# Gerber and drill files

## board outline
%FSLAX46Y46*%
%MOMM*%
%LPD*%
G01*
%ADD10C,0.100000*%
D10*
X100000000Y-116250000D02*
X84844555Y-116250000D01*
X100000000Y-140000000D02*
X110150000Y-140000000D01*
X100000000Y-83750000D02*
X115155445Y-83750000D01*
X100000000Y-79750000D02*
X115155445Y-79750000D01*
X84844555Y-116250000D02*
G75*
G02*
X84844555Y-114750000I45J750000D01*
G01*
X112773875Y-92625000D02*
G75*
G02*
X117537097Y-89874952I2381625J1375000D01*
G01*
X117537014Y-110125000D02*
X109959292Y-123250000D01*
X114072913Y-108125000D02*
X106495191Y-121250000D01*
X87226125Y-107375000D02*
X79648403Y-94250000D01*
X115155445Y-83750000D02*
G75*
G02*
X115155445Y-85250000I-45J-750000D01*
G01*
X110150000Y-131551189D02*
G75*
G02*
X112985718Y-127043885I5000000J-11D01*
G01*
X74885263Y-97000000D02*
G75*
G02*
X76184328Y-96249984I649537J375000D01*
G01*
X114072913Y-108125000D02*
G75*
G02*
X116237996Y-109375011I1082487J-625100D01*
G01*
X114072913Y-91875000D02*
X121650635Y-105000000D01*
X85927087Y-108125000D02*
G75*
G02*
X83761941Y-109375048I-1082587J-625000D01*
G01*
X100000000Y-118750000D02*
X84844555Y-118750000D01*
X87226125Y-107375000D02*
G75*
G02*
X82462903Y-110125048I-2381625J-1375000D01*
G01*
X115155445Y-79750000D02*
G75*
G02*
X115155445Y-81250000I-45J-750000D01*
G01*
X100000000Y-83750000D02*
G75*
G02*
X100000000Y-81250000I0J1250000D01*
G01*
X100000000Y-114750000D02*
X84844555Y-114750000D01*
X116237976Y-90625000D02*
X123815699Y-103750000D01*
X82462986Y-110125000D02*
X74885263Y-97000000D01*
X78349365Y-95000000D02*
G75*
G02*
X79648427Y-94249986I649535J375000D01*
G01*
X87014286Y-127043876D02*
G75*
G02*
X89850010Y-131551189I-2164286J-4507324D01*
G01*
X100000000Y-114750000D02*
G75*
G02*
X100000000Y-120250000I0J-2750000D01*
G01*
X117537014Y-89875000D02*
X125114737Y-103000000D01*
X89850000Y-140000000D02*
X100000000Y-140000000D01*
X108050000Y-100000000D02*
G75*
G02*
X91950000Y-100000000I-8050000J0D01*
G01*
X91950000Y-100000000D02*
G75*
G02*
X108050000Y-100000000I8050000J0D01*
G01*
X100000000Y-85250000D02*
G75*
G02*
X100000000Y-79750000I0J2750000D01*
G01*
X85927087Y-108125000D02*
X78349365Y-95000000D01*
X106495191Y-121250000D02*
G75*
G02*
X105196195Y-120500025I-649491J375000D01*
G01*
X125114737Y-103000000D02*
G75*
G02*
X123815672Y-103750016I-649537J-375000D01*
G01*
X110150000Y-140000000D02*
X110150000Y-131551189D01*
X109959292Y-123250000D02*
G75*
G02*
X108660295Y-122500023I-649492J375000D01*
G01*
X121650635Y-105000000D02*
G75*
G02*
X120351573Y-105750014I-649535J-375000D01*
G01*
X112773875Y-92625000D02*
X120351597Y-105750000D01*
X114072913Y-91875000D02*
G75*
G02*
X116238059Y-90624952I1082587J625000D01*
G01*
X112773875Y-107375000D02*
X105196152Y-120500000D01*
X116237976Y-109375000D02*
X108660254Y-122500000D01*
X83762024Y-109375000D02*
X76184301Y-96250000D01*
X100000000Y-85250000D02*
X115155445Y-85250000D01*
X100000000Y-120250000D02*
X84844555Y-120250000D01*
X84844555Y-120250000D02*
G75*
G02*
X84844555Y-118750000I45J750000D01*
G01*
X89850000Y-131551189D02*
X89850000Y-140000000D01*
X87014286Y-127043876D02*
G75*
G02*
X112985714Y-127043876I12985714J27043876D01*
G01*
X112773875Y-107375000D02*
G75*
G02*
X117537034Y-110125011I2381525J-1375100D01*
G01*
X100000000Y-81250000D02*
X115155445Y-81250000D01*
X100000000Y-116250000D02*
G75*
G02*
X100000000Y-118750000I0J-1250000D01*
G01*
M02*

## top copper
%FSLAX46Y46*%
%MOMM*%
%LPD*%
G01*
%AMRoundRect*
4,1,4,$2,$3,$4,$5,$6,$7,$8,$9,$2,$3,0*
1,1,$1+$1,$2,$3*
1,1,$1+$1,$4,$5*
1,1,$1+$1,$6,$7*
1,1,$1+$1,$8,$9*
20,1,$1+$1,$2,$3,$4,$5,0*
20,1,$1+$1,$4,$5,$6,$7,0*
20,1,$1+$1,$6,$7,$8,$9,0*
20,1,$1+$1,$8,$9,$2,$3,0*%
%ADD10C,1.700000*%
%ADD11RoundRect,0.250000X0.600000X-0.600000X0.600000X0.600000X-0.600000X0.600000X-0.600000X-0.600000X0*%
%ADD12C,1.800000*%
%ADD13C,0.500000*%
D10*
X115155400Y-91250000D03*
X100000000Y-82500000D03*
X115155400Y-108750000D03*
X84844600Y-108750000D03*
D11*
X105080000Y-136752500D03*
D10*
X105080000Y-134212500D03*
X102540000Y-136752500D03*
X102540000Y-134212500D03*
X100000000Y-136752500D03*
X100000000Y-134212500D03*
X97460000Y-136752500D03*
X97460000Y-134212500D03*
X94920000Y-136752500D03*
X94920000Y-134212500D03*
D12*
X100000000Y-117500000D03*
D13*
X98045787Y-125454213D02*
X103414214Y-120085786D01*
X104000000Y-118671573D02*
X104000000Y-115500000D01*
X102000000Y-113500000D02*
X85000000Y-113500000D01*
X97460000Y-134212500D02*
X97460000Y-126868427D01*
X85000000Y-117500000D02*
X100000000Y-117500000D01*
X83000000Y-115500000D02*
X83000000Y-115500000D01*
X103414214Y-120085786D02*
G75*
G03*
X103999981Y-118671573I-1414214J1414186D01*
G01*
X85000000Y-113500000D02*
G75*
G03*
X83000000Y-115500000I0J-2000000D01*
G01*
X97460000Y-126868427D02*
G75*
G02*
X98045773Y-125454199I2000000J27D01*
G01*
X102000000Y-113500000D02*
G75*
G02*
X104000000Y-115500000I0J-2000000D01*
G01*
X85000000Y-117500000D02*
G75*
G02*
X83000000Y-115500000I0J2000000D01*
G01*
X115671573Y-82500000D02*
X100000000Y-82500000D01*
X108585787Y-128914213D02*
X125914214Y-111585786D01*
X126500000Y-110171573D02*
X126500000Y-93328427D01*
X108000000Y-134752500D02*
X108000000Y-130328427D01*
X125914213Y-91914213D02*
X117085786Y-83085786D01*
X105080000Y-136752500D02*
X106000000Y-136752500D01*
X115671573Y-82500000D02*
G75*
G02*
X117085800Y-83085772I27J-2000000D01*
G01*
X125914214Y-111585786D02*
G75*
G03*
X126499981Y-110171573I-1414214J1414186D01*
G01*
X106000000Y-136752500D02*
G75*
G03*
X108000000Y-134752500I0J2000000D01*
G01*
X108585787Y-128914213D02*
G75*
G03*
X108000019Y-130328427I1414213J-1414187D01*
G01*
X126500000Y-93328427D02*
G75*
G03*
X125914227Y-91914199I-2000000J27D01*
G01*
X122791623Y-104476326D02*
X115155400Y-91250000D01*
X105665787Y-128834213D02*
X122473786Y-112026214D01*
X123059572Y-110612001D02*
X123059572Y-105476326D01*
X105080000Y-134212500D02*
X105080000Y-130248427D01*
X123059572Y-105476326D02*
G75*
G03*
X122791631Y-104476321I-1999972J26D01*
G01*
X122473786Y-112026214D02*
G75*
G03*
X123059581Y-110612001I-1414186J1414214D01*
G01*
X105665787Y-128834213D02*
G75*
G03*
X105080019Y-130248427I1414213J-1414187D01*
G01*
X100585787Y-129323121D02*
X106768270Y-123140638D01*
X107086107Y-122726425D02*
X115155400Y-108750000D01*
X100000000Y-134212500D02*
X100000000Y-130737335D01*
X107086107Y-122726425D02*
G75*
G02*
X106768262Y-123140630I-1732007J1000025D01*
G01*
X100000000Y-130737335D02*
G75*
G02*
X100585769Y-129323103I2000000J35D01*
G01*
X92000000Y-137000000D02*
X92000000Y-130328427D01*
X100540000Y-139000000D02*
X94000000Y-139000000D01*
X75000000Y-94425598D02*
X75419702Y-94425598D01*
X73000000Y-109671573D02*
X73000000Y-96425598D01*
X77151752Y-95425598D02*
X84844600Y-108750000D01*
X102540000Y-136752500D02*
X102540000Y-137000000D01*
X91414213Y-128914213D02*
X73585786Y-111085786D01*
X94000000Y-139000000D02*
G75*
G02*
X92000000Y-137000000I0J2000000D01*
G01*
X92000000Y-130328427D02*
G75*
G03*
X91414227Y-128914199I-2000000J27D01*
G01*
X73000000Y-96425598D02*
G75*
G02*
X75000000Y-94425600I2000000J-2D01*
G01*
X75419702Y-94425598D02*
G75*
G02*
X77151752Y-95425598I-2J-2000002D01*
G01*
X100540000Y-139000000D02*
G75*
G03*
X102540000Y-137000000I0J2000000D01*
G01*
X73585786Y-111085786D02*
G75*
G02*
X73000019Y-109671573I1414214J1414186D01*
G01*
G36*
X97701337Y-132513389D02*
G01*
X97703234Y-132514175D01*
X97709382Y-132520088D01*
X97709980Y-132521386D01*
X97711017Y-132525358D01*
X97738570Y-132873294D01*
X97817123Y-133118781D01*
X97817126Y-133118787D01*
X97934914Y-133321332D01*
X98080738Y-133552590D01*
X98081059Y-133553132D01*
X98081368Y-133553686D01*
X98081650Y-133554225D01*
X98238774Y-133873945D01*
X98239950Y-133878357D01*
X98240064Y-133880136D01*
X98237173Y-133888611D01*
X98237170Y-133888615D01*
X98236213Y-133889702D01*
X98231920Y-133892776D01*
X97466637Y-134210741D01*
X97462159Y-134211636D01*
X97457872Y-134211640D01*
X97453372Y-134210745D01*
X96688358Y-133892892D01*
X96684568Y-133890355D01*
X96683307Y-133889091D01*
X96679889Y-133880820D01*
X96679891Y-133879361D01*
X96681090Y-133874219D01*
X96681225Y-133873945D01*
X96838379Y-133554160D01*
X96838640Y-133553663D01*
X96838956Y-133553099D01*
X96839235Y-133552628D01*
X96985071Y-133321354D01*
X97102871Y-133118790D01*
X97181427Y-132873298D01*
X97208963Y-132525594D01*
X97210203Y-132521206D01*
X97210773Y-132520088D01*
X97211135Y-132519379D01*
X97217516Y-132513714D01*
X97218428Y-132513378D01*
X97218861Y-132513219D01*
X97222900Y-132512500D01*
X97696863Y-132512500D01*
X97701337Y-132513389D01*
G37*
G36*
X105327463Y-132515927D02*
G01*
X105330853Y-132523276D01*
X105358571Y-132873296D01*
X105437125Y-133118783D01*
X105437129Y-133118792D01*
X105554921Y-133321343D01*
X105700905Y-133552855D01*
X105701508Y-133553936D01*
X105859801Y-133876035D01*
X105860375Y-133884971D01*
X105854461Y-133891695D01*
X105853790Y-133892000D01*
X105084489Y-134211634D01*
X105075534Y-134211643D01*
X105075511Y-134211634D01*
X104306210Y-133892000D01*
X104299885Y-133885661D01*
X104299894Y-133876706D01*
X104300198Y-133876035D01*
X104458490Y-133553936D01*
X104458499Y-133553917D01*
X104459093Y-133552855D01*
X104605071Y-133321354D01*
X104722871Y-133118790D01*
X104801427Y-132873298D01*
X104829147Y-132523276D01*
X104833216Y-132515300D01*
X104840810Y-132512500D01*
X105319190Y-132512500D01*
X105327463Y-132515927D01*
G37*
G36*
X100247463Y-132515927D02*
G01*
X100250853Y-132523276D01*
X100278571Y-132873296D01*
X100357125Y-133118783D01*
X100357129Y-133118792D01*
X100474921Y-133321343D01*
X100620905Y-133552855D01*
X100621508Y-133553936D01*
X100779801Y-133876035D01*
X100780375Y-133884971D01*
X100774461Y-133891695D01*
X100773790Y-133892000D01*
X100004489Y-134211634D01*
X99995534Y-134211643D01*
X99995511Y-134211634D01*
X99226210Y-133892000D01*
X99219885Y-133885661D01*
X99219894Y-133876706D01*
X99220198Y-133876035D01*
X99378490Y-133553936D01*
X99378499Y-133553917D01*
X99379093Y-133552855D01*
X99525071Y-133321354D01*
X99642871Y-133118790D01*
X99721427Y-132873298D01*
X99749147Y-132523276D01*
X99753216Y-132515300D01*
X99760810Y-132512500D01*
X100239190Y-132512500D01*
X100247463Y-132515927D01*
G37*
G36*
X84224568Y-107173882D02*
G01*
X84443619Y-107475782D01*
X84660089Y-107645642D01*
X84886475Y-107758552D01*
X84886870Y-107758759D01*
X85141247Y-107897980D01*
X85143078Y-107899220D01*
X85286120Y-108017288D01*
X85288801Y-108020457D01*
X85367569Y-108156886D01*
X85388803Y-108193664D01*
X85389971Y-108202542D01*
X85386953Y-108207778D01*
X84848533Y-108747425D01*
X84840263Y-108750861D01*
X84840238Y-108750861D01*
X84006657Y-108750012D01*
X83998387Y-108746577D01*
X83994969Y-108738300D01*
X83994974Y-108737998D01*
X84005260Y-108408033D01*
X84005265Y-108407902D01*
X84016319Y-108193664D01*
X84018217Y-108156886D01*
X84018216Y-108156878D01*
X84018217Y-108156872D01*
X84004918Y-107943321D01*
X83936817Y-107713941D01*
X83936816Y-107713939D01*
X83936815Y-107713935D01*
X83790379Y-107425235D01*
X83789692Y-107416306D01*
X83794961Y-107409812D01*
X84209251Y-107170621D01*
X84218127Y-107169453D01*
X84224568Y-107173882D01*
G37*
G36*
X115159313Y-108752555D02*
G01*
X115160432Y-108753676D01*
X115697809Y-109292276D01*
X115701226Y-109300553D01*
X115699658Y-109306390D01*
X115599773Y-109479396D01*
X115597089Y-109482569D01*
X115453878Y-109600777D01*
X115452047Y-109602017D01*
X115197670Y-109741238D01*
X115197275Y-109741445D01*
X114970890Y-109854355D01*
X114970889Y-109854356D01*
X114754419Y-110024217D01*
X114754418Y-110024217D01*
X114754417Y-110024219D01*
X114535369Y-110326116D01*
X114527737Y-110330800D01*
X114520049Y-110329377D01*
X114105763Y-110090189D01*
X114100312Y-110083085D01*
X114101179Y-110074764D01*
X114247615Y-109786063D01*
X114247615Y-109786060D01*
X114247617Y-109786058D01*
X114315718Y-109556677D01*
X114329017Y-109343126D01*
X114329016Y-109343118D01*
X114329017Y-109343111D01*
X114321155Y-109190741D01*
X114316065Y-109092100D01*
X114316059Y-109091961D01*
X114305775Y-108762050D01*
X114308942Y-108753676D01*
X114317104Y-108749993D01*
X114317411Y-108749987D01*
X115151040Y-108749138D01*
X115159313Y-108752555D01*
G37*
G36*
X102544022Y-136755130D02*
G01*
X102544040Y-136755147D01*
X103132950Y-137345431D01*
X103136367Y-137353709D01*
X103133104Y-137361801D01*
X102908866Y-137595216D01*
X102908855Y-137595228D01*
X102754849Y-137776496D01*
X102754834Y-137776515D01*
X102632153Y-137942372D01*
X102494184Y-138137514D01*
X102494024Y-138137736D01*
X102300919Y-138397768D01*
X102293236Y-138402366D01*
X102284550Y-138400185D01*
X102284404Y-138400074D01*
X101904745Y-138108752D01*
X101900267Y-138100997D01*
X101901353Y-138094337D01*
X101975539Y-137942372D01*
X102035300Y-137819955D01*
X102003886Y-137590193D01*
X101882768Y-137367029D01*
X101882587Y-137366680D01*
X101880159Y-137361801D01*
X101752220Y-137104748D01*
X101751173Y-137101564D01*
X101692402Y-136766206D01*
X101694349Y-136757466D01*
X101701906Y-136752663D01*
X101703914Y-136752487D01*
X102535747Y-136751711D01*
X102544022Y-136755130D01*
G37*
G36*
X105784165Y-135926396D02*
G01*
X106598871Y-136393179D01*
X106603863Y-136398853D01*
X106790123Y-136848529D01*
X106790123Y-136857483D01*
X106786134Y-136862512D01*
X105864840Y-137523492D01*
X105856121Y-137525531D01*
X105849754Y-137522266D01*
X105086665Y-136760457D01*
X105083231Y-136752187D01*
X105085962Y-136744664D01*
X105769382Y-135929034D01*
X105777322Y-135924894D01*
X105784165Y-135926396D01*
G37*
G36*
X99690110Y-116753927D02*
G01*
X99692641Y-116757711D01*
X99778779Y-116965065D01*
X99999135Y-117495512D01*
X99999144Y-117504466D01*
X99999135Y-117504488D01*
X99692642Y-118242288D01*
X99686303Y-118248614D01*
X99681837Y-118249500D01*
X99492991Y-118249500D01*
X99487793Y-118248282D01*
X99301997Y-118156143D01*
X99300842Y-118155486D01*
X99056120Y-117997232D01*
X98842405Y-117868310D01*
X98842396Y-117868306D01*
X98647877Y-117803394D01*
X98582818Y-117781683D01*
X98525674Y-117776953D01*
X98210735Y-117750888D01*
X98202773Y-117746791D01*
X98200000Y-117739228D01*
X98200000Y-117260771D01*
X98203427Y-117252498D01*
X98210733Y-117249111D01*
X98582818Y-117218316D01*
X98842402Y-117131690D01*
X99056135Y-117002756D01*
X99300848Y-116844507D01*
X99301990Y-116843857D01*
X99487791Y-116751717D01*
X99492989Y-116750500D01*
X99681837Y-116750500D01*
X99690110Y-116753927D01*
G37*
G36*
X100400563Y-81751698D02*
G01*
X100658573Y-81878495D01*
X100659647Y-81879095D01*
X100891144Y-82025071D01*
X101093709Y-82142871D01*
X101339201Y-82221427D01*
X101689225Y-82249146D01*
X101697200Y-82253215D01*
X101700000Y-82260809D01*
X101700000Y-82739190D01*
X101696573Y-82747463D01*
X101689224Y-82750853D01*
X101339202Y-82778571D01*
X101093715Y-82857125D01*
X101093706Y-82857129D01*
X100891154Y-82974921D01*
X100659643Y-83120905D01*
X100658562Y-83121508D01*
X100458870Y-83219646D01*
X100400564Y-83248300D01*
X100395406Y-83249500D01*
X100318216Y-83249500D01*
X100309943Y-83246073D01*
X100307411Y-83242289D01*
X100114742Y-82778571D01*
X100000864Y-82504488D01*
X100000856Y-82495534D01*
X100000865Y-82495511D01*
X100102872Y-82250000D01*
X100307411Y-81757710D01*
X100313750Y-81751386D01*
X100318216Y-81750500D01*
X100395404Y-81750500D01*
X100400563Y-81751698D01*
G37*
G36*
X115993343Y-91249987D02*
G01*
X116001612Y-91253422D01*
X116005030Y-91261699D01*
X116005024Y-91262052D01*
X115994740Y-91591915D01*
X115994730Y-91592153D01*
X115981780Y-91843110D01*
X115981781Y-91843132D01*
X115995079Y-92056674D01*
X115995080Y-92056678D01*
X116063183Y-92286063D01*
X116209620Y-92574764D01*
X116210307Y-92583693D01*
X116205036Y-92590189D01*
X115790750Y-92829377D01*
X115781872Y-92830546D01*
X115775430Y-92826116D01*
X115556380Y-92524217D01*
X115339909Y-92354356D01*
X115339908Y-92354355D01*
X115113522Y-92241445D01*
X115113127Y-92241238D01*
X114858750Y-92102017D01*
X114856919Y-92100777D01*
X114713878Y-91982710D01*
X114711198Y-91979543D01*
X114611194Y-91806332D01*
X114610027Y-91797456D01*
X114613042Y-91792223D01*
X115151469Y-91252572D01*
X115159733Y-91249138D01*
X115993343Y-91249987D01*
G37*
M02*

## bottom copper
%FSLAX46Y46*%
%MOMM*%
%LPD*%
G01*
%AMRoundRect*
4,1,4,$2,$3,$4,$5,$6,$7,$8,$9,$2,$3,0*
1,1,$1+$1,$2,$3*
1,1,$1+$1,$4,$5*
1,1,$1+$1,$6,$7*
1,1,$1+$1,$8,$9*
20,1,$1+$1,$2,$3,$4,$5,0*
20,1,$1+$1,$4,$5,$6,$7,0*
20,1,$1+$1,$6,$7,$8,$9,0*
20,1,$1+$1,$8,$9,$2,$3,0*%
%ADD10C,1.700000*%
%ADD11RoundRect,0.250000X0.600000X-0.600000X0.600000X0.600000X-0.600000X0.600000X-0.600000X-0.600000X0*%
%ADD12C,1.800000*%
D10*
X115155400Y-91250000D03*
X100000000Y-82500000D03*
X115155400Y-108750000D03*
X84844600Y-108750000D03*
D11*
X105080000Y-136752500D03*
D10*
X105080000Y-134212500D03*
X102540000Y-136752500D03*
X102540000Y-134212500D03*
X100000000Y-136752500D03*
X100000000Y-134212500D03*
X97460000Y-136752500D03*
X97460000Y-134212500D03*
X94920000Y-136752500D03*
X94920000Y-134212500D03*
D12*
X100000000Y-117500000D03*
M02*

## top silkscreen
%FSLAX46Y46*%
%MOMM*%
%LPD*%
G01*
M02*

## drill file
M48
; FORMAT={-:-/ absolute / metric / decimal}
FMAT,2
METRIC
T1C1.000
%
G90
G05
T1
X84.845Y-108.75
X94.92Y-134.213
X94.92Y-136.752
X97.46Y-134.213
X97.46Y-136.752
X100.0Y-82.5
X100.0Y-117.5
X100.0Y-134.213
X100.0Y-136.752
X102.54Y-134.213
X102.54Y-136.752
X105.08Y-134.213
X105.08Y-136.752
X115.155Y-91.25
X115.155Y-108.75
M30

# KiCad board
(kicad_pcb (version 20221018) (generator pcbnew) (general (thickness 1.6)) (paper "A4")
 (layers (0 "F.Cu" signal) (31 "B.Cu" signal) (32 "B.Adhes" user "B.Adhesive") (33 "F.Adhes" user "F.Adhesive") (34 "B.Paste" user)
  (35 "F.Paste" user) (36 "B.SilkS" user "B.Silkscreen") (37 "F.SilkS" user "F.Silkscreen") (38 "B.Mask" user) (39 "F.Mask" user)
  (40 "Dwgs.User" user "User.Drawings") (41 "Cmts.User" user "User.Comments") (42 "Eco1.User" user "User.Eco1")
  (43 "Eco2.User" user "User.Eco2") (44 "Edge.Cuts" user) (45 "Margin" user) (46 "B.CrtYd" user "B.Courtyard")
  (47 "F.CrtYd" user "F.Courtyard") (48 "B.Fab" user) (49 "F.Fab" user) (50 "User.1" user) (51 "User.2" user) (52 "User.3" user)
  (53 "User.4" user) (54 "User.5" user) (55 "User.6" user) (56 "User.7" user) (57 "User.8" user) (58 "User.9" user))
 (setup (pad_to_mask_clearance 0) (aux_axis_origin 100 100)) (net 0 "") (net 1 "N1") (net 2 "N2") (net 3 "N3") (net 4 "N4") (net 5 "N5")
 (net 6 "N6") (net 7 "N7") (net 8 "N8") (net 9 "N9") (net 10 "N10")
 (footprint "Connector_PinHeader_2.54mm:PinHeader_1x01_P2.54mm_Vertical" (layer "B.Cu") (at 115.1554 91.25 180)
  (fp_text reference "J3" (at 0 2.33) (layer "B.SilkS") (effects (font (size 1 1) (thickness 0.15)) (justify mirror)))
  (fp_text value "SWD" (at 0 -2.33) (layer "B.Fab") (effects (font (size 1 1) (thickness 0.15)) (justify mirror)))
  (pad "1" thru_hole circle (at 0 0 180) (size 1.7 1.7) (drill 1) (layers "*.Cu" "*.Mask") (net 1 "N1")))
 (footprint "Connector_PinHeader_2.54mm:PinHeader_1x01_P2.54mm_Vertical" (layer "B.Cu") (at 100 82.5 180)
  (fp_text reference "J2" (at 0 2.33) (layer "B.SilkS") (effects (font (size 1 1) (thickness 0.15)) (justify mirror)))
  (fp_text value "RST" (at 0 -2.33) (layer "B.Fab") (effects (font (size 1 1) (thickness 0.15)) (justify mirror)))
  (pad "1" thru_hole circle (at 0 0 180) (size 1.7 1.7) (drill 1) (layers "*.Cu" "*.Mask") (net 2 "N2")))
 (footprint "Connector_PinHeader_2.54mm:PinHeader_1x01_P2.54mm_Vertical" (layer "B.Cu") (at 115.1554 108.75 180)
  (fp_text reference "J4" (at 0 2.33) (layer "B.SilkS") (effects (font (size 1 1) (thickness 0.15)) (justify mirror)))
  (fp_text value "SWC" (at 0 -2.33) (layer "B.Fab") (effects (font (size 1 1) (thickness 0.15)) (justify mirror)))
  (pad "1" thru_hole circle (at 0 0 180) (size 1.7 1.7) (drill 1) (layers "*.Cu" "*.Mask") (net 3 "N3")))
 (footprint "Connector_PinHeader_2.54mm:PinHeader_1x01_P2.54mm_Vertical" (layer "B.Cu") (at 84.8446 108.75 180)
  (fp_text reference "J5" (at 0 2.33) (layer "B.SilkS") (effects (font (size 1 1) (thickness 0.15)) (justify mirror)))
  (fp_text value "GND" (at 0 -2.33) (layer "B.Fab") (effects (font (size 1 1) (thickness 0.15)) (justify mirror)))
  (pad "1" thru_hole circle (at 0 0 180) (size 1.7 1.7) (drill 1) (layers "*.Cu" "*.Mask") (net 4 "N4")))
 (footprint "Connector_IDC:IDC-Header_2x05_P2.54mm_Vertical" (layer "B.Cu") (at 105.08 136.7525 90)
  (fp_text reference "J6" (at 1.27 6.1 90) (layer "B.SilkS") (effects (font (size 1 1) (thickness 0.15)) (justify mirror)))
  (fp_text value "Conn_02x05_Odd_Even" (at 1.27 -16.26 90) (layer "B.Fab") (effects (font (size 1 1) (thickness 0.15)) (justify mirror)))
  (pad "1" thru_hole roundrect (at 0 0 90) (size 1.7 1.7) (drill 1) (layers "*.Cu" "*.Mask") (roundrect_rratio 0.1470588235) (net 2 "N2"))
  (pad "2" thru_hole circle (at 2.54 0 90) (size 1.7 1.7) (drill 1) (layers "*.Cu" "*.Mask") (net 1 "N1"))
  (pad "3" thru_hole circle (at 0 -2.54 90) (size 1.7 1.7) (drill 1) (layers "*.Cu" "*.Mask") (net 4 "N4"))
  (pad "4" thru_hole circle (at 2.54 -2.54 90) (size 1.7 1.7) (drill 1) (layers "*.Cu" "*.Mask") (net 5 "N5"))
  (pad "5" thru_hole circle (at 0 -5.08 90) (size 1.7 1.7) (drill 1) (layers "*.Cu" "*.Mask") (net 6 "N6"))
  (pad "6" thru_hole circle (at 2.54 -5.08 90) (size 1.7 1.7) (drill 1) (layers "*.Cu" "*.Mask") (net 3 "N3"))
  (pad "7" thru_hole circle (at 0 -7.62 90) (size 1.7 1.7) (drill 1) (layers "*.Cu" "*.Mask") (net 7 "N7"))
  (pad "8" thru_hole circle (at 2.54 -7.62 90) (size 1.7 1.7) (drill 1) (layers "*.Cu" "*.Mask") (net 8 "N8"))
  (pad "9" thru_hole circle (at 0 -10.16 90) (size 1.7 1.7) (drill 1) (layers "*.Cu" "*.Mask") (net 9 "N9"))
  (pad "10" thru_hole circle (at 2.54 -10.16 90) (size 1.7 1.7) (drill 1) (layers "*.Cu" "*.Mask") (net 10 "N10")))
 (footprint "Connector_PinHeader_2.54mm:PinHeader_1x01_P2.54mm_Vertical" (layer "B.Cu") (at 100 117.5 180)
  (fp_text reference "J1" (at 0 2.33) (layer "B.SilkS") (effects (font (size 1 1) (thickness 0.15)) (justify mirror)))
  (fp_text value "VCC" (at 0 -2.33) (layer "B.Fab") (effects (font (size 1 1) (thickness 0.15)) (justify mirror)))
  (pad "1" thru_hole circle (at 0 0 180) (size 1.8 1.8) (drill 1) (layers "*.Cu" "*.Mask") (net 8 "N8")))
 (gr_line (start 100 116.25) (end 84.844555 116.25) (stroke (width 0.1) (type solid)) (layer "Edge.Cuts"))
 (gr_line (start 100 140) (end 110.15 140) (stroke (width 0.1) (type solid)) (layer "Edge.Cuts"))
 (gr_line (start 100 83.75) (end 115.155445 83.75) (stroke (width 0.1) (type solid)) (layer "Edge.Cuts"))
 (gr_line (start 100 79.75) (end 115.155445 79.75) (stroke (width 0.1) (type solid)) (layer "Edge.Cuts"))
 (gr_arc (start 84.844555 116.25) (mid 84.0946 115.5) (end 84.844555 114.75) (stroke (width 0.1) (type solid)) (layer "Edge.Cuts"))
 (gr_arc (start 112.773875 92.625) (mid 113.780419 88.868464) (end 117.537014 89.875) (stroke (width 0.1) (type solid)) (layer "Edge.Cuts"))
 (gr_line (start 117.537014 110.125) (end 109.959292 123.25) (stroke (width 0.1) (type solid)) (layer "Edge.Cuts"))
 (gr_line (start 114.072913 108.125) (end 106.495191 121.25) (stroke (width 0.1) (type solid)) (layer "Edge.Cuts"))
 (gr_line (start 87.226125 107.375) (end 79.648403 94.25) (stroke (width 0.1) (type solid)) (layer "Edge.Cuts"))
 (gr_arc (start 115.155445 83.75) (mid 115.9054 84.5) (end 115.155445 85.25) (stroke (width 0.1) (type solid)) (layer "Edge.Cuts"))
 (gr_arc (start 110.15 131.551189) (mid 110.917899 128.888622) (end 112.985714 127.043876) (stroke (width 0.1) (type solid))
  (layer "Edge.Cuts"))
 (gr_arc (start 74.885263 97) (mid 75.159792 95.975468) (end 76.184301 96.25) (stroke (width 0.1) (type solid)) (layer "Edge.Cuts"))
 (gr_arc (start 114.072913 108.125) (mid 115.780381 107.667502) (end 116.237976 109.375) (stroke (width 0.1) (type solid))
  (layer "Edge.Cuts"))
 (gr_line (start 114.072913 91.875) (end 121.650635 105) (stroke (width 0.1) (type solid)) (layer "Edge.Cuts"))
 (gr_arc (start 85.927087 108.125) (mid 85.469581 109.832498) (end 83.762024 109.375) (stroke (width 0.1) (type solid)) (layer "Edge.Cuts"))
 (gr_line (start 100 118.75) (end 84.844555 118.75) (stroke (width 0.1) (type solid)) (layer "Edge.Cuts"))
 (gr_arc (start 87.226125 107.375) (mid 86.219581 111.131536) (end 82.462986 110.125) (stroke (width 0.1) (type solid)) (layer "Edge.Cuts"))
 (gr_arc (start 115.155445 79.75) (mid 115.9054 80.5) (end 115.155445 81.25) (stroke (width 0.1) (type solid)) (layer "Edge.Cuts"))
 (gr_arc (start 100 83.75) (mid 98.75 82.5) (end 100 81.25) (stroke (width 0.1) (type solid)) (layer "Edge.Cuts"))
 (gr_line (start 100 114.75) (end 84.844555 114.75) (stroke (width 0.1) (type solid)) (layer "Edge.Cuts"))
 (gr_line (start 116.237976 90.625) (end 123.815699 103.75) (stroke (width 0.1) (type solid)) (layer "Edge.Cuts"))
 (gr_line (start 82.462986 110.125) (end 74.885263 97) (stroke (width 0.1) (type solid)) (layer "Edge.Cuts"))
 (gr_arc (start 78.349365 95) (mid 78.623893 93.975469) (end 79.648403 94.25) (stroke (width 0.1) (type solid)) (layer "Edge.Cuts"))
 (gr_arc (start 87.014286 127.043876) (mid 89.08211 128.888617) (end 89.85 131.551189) (stroke (width 0.1) (type solid)) (layer "Edge.Cuts"))
 (gr_arc (start 100 114.75) (mid 102.75 117.5) (end 100 120.25) (stroke (width 0.1) (type solid)) (layer "Edge.Cuts"))
 (gr_line (start 117.537014 89.875) (end 125.114737 103) (stroke (width 0.1) (type solid)) (layer "Edge.Cuts"))
 (gr_line (start 89.85 140) (end 100 140) (stroke (width 0.1) (type solid)) (layer "Edge.Cuts"))
 (gr_circle (center 100 100) (end 108.05 100) (stroke (width 0.1) (type solid)) (fill none) (layer "Edge.Cuts"))
 (gr_arc (start 100 85.25) (mid 97.25 82.5) (end 100 79.75) (stroke (width 0.1) (type solid)) (layer "Edge.Cuts"))
 (gr_line (start 85.927087 108.125) (end 78.349365 95) (stroke (width 0.1) (type solid)) (layer "Edge.Cuts"))
 (gr_arc (start 106.495191 121.25) (mid 105.470712 121.524498) (end 105.196152 120.5) (stroke (width 0.1) (type solid)) (layer "Edge.Cuts"))
 (gr_arc (start 125.114737 103) (mid 124.840208 104.024532) (end 123.815699 103.75) (stroke (width 0.1) (type solid)) (layer "Edge.Cuts"))
 (gr_line (start 110.15 140) (end 110.15 131.551189) (stroke (width 0.1) (type solid)) (layer "Edge.Cuts"))
 (gr_arc (start 109.959292 123.25) (mid 108.934812 123.524499) (end 108.660254 122.5) (stroke (width 0.1) (type solid)) (layer "Edge.Cuts"))
 (gr_arc (start 121.650635 105) (mid 121.376107 106.024531) (end 120.351597 105.75) (stroke (width 0.1) (type solid)) (layer "Edge.Cuts"))
 (gr_line (start 112.773875 92.625) (end 120.351597 105.75) (stroke (width 0.1) (type solid)) (layer "Edge.Cuts"))
 (gr_arc (start 114.072913 91.875) (mid 114.530419 90.167502) (end 116.237976 90.625) (stroke (width 0.1) (type solid)) (layer "Edge.Cuts"))
 (gr_line (start 112.773875 107.375) (end 105.196152 120.5) (stroke (width 0.1) (type solid)) (layer "Edge.Cuts"))
 (gr_line (start 116.237976 109.375) (end 108.660254 122.5) (stroke (width 0.1) (type solid)) (layer "Edge.Cuts"))
 (gr_line (start 83.762024 109.375) (end 76.184301 96.25) (stroke (width 0.1) (type solid)) (layer "Edge.Cuts"))
 (gr_line (start 100 85.25) (end 115.155445 85.25) (stroke (width 0.1) (type solid)) (layer "Edge.Cuts"))
 (gr_line (start 100 120.25) (end 84.844555 120.25) (stroke (width 0.1) (type solid)) (layer "Edge.Cuts"))
 (gr_arc (start 84.844555 120.25) (mid 84.0946 119.5) (end 84.844555 118.75) (stroke (width 0.1) (type solid)) (layer "Edge.Cuts"))
 (gr_line (start 89.85 131.551189) (end 89.85 140) (stroke (width 0.1) (type solid)) (layer "Edge.Cuts"))
 (gr_arc (start 87.014286 127.043876) (mid 100 70) (end 112.985714 127.043876) (stroke (width 0.1) (type solid)) (layer "Edge.Cuts"))
 (gr_arc (start 112.773875 107.375) (mid 116.530381 106.368464) (end 117.537014 110.125) (stroke (width 0.1) (type solid))
  (layer "Edge.Cuts"))
 (gr_line (start 100 81.25) (end 115.155445 81.25) (stroke (width 0.1) (type solid)) (layer "Edge.Cuts"))
 (gr_arc (start 100 116.25) (mid 101.25 117.5) (end 100 118.75) (stroke (width 0.1) (type solid)) (layer "Edge.Cuts"))
 (segment (start 98.045787 125.454213) (end 103.414214 120.085786) (width 0.5) (layer "F.Cu") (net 8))
 (segment (start 104 118.671573) (end 104 115.5) (width 0.5) (layer "F.Cu") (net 8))
 (segment (start 102 113.5) (end 85 113.5) (width 0.5) (layer "F.Cu") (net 8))
 (segment (start 97.46 134.2125) (end 97.46 126.868427) (width 0.5) (layer "F.Cu") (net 8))
 (segment (start 85 117.5) (end 100 117.5) (width 0.5) (layer "F.Cu") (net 8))
 (segment (start 83 115.5) (end 83 115.5) (width 0.5) (layer "F.Cu") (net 8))
 (arc (start 103.414214 120.085786) (mid 103.847759 119.43694) (end 104 118.671573) (width 0.5) (layer "F.Cu") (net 8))
 (arc (start 85 113.5) (mid 83.585786 114.085786) (end 83 115.5) (width 0.5) (layer "F.Cu") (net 8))
 (arc (start 97.46 126.868427) (mid 97.612241 126.10306) (end 98.045787 125.454213) (width 0.5) (layer "F.Cu") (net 8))
 (arc (start 102 113.5) (mid 103.414214 114.085786) (end 104 115.5) (width 0.5) (layer "F.Cu") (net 8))
 (arc (start 85 117.5) (mid 83.585786 116.914214) (end 83 115.5) (width 0.5) (layer "F.Cu") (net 8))
 (segment (start 115.671573 82.5) (end 100 82.5) (width 0.5) (layer "F.Cu") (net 2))
 (segment (start 108.585787 128.914213) (end 125.914214 111.585786) (width 0.5) (layer "F.Cu") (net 2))
 (segment (start 126.5 110.171573) (end 126.5 93.328427) (width 0.5) (layer "F.Cu") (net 2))
 (segment (start 108 134.7525) (end 108 130.328427) (width 0.5) (layer "F.Cu") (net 2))
 (segment (start 125.914213 91.914213) (end 117.085786 83.085786) (width 0.5) (layer "F.Cu") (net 2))
 (segment (start 105.08 136.7525) (end 106 136.7525) (width 0.5) (layer "F.Cu") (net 2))
 (arc (start 115.671573 82.5) (mid 116.43694 82.652241) (end 117.085786 83.085786) (width 0.5) (layer "F.Cu") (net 2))
 (arc (start 125.914214 111.585786) (mid 126.347759 110.93694) (end 126.5 110.171573) (width 0.5) (layer "F.Cu") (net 2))
 (arc (start 106 136.7525) (mid 107.414214 136.166714) (end 108 134.7525) (width 0.5) (layer "F.Cu") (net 2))
 (arc (start 108.585787 128.914213) (mid 108.152241 129.56306) (end 108 130.328427) (width 0.5) (layer "F.Cu") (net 2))
 (arc (start 126.5 93.328427) (mid 126.347759 92.56306) (end 125.914213 91.914213) (width 0.5) (layer "F.Cu") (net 2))
 (segment (start 122.791623 104.476326) (end 115.1554 91.25) (width 0.5) (layer "F.Cu") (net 1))
 (segment (start 105.665787 128.834213) (end 122.473786 112.026214) (width 0.5) (layer "F.Cu") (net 1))
 (segment (start 123.059572 110.612001) (end 123.059572 105.476326) (width 0.5) (layer "F.Cu") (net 1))
 (segment (start 105.08 134.2125) (end 105.08 130.248427) (width 0.5) (layer "F.Cu") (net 1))
 (arc (start 123.059572 105.476326) (mid 122.991424 104.958688) (end 122.791623 104.476326) (width 0.5) (layer "F.Cu") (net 1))
 (arc (start 122.473786 112.026214) (mid 122.907331 111.377368) (end 123.059572 110.612001) (width 0.5) (layer "F.Cu") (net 1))
 (arc (start 105.665787 128.834213) (mid 105.232241 129.48306) (end 105.08 130.248427) (width 0.5) (layer "F.Cu") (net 1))
 (segment (start 100.585787 129.323121) (end 106.76827 123.140638) (width 0.5) (layer "F.Cu") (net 3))
 (segment (start 107.086107 122.726425) (end 115.1554 108.75) (width 0.5) (layer "F.Cu") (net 3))
 (segment (start 100 134.2125) (end 100 130.737335) (width 0.5) (layer "F.Cu") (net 3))
 (arc (start 107.086107 122.726425) (mid 106.940763 122.943948) (end 106.76827 123.140638) (width 0.5) (layer "F.Cu") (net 3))
 (arc (start 100 130.737335) (mid 100.152241 129.971968) (end 100.585787 129.323121) (width 0.5) (layer "F.Cu") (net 3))
 (segment (start 92 137) (end 92 130.328427) (width 0.5) (layer "F.Cu") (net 4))
 (segment (start 100.54 139) (end 94 139) (width 0.5) (layer "F.Cu") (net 4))
 (segment (start 75 94.425598) (end 75.419702 94.425598) (width 0.5) (layer "F.Cu") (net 4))
 (segment (start 73 109.671573) (end 73 96.425598) (width 0.5) (layer "F.Cu") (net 4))
 (segment (start 77.151752 95.425598) (end 84.8446 108.75) (width 0.5) (layer "F.Cu") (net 4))
 (segment (start 102.54 136.7525) (end 102.54 137) (width 0.5) (layer "F.Cu") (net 4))
 (segment (start 91.414213 128.914213) (end 73.585786 111.085786) (width 0.5) (layer "F.Cu") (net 4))
 (arc (start 94 139) (mid 92.585786 138.414214) (end 92 137) (width 0.5) (layer "F.Cu") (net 4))
 (arc (start 92 130.328427) (mid 91.847759 129.56306) (end 91.414213 128.914213) (width 0.5) (layer "F.Cu") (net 4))
 (arc (start 73 96.425598) (mid 73.585786 95.011384) (end 75 94.425598) (width 0.5) (layer "F.Cu") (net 4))
 (arc (start 75.419702 94.425598) (mid 76.419702 94.693547) (end 77.151752 95.425598) (width 0.5) (layer "F.Cu") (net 4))
 (arc (start 100.54 139) (mid 101.954214 138.414214) (end 102.54 137) (width 0.5) (layer "F.Cu") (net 4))
 (arc (start 73.585786 111.085786) (mid 73.152241 110.43694) (end 73 109.671573) (width 0.5) (layer "F.Cu") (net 4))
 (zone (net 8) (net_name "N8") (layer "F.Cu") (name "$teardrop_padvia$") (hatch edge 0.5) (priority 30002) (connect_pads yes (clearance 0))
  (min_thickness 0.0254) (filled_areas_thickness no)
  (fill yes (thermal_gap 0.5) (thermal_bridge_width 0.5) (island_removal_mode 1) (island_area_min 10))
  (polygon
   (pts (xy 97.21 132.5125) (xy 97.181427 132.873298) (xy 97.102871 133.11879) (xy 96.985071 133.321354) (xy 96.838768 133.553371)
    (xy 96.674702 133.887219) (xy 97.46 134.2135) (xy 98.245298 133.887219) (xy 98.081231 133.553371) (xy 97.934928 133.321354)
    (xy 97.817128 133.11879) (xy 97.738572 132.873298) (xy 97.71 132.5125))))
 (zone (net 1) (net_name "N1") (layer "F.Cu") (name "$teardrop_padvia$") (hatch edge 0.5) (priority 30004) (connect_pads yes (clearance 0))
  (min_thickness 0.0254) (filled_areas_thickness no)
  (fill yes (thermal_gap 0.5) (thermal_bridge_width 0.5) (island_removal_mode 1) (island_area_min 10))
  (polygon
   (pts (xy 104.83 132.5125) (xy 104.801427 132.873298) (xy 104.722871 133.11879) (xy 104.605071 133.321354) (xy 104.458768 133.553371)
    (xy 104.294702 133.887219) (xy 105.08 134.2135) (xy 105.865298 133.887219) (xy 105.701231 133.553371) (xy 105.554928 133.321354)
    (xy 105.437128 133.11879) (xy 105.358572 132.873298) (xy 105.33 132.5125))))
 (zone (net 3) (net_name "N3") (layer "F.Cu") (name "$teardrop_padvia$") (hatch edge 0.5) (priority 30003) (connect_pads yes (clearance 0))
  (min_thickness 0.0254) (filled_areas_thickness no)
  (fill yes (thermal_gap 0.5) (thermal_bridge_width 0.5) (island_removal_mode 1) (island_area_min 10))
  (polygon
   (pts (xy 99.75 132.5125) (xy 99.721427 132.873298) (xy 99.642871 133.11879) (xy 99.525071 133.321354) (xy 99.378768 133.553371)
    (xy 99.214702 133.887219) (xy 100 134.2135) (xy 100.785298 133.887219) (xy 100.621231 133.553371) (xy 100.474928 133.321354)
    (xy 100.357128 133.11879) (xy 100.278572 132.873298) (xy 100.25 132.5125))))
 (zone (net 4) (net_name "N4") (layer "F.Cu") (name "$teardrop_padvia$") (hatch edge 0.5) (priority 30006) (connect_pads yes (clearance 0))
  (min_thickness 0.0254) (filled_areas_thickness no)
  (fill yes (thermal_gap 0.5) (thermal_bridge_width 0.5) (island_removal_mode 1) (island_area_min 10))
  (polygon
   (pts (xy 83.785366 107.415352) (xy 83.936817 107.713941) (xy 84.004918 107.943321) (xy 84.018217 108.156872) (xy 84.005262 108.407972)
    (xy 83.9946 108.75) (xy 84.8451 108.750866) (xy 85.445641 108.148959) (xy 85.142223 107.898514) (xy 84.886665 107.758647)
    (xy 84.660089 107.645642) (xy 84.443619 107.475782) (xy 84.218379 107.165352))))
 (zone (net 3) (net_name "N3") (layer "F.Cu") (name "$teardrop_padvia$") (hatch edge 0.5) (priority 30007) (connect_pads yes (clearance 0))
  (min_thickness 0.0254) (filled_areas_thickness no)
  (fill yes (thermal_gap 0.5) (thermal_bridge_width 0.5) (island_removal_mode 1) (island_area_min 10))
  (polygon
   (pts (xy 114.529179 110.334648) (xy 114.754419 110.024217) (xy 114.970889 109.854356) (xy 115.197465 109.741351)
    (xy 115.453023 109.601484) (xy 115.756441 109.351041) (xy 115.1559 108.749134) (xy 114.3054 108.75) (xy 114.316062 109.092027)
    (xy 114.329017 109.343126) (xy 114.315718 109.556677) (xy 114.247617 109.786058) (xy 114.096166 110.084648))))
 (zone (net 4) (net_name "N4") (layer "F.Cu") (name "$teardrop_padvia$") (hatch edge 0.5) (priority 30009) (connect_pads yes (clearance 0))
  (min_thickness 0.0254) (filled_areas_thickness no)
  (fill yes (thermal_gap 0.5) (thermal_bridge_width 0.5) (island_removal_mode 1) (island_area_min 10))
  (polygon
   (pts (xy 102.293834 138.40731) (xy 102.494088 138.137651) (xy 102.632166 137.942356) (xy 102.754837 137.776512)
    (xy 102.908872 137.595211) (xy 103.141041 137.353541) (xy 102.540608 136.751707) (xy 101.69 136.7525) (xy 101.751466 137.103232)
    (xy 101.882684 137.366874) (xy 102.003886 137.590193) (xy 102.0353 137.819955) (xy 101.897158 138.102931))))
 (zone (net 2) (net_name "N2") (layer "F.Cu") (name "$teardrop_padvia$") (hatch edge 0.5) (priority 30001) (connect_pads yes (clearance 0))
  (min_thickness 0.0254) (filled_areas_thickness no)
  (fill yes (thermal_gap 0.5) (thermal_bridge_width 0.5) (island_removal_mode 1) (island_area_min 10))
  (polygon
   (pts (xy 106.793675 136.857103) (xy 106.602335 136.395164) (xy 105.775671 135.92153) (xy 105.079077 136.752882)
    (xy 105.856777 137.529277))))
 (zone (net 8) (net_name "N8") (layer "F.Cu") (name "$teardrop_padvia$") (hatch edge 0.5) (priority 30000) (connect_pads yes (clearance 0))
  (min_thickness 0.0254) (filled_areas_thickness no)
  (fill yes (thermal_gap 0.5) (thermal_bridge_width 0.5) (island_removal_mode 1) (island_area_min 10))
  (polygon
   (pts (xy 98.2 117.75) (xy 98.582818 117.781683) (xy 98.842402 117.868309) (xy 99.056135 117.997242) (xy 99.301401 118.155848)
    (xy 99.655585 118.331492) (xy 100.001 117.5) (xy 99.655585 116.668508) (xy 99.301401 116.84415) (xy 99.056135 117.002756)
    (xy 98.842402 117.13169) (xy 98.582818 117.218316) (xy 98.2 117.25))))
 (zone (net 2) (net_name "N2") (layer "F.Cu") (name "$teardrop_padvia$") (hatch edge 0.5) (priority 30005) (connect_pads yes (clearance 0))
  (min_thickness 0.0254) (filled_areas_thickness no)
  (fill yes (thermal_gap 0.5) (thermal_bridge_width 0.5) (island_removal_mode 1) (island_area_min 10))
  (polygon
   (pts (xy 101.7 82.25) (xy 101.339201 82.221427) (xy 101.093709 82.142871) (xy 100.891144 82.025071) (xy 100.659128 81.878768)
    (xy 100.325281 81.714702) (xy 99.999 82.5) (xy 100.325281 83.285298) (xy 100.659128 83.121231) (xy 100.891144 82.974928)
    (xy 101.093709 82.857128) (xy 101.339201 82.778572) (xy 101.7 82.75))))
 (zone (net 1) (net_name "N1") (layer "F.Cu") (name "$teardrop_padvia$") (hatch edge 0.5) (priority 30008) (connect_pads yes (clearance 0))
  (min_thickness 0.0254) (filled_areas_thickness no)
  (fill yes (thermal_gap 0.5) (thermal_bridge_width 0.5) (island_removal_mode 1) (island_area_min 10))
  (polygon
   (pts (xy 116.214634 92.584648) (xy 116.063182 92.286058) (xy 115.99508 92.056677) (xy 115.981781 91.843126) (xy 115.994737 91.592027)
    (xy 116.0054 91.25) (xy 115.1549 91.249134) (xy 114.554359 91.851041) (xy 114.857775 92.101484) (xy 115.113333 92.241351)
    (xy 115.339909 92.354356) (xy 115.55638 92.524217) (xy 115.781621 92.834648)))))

